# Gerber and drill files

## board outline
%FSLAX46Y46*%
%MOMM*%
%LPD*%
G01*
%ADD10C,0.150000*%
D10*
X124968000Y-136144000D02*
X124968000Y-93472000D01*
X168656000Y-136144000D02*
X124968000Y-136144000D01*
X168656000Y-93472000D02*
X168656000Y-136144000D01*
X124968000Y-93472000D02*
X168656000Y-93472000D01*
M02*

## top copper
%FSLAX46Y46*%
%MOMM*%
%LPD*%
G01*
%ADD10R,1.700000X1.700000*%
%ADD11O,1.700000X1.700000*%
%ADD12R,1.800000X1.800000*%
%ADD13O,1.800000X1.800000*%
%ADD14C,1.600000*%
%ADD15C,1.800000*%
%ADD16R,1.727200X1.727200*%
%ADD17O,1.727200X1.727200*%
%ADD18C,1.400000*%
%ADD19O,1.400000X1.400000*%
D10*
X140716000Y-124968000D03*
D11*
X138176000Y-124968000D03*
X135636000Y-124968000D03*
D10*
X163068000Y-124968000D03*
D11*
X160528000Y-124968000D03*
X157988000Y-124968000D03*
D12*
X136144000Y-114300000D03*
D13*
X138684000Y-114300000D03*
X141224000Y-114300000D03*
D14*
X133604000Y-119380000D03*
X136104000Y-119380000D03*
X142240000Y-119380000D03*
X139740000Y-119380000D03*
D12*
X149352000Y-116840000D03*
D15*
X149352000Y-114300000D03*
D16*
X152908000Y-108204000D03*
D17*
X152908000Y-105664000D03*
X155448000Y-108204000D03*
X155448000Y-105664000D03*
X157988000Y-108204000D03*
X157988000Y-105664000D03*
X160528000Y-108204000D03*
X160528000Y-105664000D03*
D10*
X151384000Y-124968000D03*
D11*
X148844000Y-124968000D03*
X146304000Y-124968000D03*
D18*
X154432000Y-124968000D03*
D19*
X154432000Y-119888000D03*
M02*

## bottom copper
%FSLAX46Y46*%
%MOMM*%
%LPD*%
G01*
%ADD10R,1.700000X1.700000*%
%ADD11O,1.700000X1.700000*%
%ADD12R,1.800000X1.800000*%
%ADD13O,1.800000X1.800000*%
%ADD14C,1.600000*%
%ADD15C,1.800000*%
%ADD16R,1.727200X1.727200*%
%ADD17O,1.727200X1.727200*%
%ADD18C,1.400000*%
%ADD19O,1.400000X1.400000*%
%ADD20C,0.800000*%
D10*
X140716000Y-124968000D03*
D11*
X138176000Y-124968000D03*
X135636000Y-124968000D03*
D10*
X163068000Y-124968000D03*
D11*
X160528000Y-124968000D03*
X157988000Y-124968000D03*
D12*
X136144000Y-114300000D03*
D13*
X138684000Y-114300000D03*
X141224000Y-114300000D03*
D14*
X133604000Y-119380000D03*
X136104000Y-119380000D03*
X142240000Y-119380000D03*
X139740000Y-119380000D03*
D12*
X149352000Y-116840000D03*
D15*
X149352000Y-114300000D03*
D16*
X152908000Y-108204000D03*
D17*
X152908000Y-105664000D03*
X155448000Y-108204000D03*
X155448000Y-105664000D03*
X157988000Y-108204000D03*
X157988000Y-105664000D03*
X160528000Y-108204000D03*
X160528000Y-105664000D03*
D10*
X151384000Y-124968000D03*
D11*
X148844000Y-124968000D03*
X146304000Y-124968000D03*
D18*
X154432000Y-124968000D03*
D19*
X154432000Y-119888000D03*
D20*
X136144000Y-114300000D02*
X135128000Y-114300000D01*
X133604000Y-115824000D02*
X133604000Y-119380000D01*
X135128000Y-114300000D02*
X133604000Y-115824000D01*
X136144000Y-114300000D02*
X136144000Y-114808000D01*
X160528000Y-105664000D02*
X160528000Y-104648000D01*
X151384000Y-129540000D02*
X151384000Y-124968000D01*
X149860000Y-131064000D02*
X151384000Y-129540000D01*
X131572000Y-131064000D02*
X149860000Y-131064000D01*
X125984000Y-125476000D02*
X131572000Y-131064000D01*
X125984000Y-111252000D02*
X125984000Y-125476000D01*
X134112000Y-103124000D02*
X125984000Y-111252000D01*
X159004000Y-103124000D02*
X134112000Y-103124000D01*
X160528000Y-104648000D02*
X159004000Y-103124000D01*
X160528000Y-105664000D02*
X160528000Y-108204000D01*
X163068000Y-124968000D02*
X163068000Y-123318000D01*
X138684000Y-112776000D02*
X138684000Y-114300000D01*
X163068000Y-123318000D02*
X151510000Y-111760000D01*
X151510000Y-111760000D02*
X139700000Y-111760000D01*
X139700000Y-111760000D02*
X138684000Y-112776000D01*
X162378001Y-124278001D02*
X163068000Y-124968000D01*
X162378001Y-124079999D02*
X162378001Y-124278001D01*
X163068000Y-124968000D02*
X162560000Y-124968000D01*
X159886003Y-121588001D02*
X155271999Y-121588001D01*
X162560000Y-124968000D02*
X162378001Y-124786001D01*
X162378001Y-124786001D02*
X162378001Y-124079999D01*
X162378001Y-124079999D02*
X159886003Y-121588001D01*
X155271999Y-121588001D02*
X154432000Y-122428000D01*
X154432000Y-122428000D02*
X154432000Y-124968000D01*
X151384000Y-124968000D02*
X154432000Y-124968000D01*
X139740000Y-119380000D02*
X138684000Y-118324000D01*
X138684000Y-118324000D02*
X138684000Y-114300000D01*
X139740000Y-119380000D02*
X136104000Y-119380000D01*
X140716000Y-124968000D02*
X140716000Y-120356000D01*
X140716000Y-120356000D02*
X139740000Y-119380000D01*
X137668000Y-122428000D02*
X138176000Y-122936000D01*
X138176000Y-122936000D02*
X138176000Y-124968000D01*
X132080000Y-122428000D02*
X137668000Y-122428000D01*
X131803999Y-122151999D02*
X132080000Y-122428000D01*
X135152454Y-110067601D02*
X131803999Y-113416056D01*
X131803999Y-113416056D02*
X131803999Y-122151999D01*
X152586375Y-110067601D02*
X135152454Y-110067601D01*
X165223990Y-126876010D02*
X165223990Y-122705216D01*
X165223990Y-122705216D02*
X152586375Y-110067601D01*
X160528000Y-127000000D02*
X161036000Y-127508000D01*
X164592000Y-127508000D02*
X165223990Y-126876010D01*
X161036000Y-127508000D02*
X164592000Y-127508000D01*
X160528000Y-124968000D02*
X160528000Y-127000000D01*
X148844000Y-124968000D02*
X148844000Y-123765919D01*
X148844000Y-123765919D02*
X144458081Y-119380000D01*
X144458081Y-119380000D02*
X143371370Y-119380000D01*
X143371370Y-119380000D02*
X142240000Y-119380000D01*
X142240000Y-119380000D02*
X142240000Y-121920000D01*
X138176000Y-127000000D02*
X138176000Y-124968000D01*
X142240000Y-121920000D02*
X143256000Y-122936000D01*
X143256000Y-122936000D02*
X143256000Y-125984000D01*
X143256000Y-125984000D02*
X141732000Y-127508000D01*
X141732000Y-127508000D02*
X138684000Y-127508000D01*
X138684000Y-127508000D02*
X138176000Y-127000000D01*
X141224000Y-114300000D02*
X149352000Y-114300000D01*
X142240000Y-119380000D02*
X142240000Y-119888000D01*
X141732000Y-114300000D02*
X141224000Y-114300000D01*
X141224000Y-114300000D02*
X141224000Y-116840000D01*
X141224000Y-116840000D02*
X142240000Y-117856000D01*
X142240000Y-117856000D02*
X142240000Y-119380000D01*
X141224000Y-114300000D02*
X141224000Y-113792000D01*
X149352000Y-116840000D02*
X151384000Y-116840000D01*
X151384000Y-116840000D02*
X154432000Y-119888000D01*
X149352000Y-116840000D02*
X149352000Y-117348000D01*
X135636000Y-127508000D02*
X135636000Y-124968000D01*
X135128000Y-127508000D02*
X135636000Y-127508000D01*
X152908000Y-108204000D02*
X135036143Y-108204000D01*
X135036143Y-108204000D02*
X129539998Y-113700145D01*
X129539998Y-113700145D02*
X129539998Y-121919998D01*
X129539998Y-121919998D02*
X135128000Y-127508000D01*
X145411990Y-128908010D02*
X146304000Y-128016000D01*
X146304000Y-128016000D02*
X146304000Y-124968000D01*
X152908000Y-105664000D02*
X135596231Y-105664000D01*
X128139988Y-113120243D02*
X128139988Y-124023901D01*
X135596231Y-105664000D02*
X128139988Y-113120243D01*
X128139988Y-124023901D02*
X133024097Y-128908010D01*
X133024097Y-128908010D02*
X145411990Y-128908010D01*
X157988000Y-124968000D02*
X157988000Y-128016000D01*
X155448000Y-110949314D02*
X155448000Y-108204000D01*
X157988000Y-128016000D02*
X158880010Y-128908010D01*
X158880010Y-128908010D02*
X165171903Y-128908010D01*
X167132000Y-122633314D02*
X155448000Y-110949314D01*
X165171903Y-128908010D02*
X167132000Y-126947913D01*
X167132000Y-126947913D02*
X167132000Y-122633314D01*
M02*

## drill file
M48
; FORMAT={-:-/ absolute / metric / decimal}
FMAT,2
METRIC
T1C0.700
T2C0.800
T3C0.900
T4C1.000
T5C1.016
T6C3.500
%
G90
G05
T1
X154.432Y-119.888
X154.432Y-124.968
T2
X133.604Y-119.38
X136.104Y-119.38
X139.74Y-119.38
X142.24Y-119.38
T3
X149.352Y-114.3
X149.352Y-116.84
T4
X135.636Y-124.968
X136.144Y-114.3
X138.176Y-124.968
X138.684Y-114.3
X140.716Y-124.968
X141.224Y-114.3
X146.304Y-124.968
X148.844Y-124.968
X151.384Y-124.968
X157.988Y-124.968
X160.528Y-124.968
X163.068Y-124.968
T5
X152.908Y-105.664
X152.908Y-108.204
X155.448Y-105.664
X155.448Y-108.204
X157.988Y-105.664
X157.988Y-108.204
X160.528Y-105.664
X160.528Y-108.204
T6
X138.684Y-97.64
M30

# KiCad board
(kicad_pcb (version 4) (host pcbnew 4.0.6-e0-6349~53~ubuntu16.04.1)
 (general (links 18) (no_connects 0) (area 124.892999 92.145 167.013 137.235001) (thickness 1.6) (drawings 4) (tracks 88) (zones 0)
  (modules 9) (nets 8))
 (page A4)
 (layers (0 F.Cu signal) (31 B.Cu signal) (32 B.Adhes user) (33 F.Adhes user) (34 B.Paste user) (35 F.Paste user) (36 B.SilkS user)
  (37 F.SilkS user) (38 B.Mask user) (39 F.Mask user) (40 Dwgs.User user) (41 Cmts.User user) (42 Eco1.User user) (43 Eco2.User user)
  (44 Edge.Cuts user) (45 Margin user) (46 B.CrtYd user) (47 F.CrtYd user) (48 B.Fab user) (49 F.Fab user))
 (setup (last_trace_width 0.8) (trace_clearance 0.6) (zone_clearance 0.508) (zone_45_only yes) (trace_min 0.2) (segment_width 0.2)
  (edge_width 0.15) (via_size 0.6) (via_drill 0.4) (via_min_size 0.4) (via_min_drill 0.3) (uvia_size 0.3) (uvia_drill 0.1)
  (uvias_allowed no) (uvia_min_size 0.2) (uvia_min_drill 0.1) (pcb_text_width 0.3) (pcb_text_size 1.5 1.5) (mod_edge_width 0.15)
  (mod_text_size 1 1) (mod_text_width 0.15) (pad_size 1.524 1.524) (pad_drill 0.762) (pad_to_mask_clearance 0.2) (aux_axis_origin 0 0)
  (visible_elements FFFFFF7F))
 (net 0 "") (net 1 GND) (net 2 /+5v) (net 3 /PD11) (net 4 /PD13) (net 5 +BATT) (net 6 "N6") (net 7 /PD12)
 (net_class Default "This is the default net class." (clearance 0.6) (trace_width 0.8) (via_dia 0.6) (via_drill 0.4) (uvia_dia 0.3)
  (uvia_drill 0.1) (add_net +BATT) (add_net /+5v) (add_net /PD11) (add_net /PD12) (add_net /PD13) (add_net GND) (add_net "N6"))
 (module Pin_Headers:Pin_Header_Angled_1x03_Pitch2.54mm (layer F.Cu) (at 140.716 124.968 270)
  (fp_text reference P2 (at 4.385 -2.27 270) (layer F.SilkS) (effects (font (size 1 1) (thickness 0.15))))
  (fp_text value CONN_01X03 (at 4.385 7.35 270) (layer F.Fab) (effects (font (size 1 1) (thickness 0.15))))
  (pad 1 thru_hole rect (at 0 0 270) (size 1.7 1.7) (drill 1) (layers *.Cu *.Mask) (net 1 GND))
  (pad 2 thru_hole oval (at 0 2.54 270) (size 1.7 1.7) (drill 1) (layers *.Cu *.Mask) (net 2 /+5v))
  (pad 3 thru_hole oval (at 0 5.08 270) (size 1.7 1.7) (drill 1) (layers *.Cu *.Mask) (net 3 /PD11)))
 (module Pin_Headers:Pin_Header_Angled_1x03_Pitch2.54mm (layer F.Cu) (at 163.068 124.968 270)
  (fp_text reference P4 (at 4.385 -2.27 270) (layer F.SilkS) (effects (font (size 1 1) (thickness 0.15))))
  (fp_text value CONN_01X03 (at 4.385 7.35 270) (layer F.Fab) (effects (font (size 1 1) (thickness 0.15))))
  (pad 1 thru_hole rect (at 0 0 270) (size 1.7 1.7) (drill 1) (layers *.Cu *.Mask) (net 1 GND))
  (pad 2 thru_hole oval (at 0 2.54 270) (size 1.7 1.7) (drill 1) (layers *.Cu *.Mask) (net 2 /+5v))
  (pad 3 thru_hole oval (at 0 5.08 270) (size 1.7 1.7) (drill 1) (layers *.Cu *.Mask) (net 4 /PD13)))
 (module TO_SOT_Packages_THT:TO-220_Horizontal (layer F.Cu) (at 136.144 114.3)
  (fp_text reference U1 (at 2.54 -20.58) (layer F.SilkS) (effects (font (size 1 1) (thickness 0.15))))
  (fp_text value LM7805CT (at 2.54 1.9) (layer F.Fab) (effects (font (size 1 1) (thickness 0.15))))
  (pad 0 np_thru_hole oval (at 2.54 -16.66) (size 3.5 3.5) (drill 3.5) (layers *.Cu *.Mask))
  (pad 1 thru_hole rect (at 0 0) (size 1.8 1.8) (drill 1) (layers *.Cu *.Mask) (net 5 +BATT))
  (pad 2 thru_hole oval (at 2.54 0) (size 1.8 1.8) (drill 1) (layers *.Cu *.Mask) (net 1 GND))
  (pad 3 thru_hole oval (at 5.08 0) (size 1.8 1.8) (drill 1) (layers *.Cu *.Mask) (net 2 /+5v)))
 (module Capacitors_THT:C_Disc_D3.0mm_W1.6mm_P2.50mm (layer F.Cu) (at 133.604 119.38)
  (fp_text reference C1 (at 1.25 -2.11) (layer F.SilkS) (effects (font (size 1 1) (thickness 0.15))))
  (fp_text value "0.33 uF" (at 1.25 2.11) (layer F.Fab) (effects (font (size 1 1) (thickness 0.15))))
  (pad 1 thru_hole circle (at 0 0) (size 1.6 1.6) (drill 0.8) (layers *.Cu *.Mask) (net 5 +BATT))
  (pad 2 thru_hole circle (at 2.5 0) (size 1.6 1.6) (drill 0.8) (layers *.Cu *.Mask) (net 1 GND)))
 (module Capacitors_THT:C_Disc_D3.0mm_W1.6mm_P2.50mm (layer F.Cu) (at 142.24 119.38 180)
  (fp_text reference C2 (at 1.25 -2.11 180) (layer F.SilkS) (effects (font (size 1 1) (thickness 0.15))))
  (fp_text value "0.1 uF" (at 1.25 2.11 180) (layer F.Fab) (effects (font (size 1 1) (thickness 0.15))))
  (pad 1 thru_hole circle (at 0 0 180) (size 1.6 1.6) (drill 0.8) (layers *.Cu *.Mask) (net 2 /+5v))
  (pad 2 thru_hole circle (at 2.5 0 180) (size 1.6 1.6) (drill 0.8) (layers *.Cu *.Mask) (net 1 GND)))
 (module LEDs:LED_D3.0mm (layer F.Cu) (at 149.352 116.84 90)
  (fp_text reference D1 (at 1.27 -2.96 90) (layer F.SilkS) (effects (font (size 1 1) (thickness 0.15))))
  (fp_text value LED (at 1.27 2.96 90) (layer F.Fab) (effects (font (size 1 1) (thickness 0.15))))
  (pad 1 thru_hole rect (at 0 0 90) (size 1.8 1.8) (drill 0.9) (layers *.Cu *.Mask) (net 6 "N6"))
  (pad 2 thru_hole circle (at 2.54 0 90) (size 1.8 1.8) (drill 0.9) (layers *.Cu *.Mask) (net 2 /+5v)))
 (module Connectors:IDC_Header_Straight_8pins (layer F.Cu) (at 152.908 108.204)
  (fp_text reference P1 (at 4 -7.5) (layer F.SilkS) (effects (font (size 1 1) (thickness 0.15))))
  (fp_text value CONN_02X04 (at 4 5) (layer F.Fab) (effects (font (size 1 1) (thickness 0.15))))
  (pad 1 thru_hole rect (at 0 0) (size 1.7272 1.7272) (drill 1.016) (layers *.Cu *.Mask) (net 3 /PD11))
  (pad 2 thru_hole oval (at 0 -2.54) (size 1.7272 1.7272) (drill 1.016) (layers *.Cu *.Mask) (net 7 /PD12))
  (pad 3 thru_hole oval (at 2.54 0) (size 1.7272 1.7272) (drill 1.016) (layers *.Cu *.Mask) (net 4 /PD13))
  (pad 4 thru_hole oval (at 2.54 -2.54) (size 1.7272 1.7272) (drill 1.016) (layers *.Cu *.Mask))
  (pad 5 thru_hole oval (at 5.08 0) (size 1.7272 1.7272) (drill 1.016) (layers *.Cu *.Mask))
  (pad 6 thru_hole oval (at 5.08 -2.54) (size 1.7272 1.7272) (drill 1.016) (layers *.Cu *.Mask))
  (pad 7 thru_hole oval (at 7.62 0) (size 1.7272 1.7272) (drill 1.016) (layers *.Cu *.Mask) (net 1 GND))
  (pad 8 thru_hole oval (at 7.62 -2.54) (size 1.7272 1.7272) (drill 1.016) (layers *.Cu *.Mask) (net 1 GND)))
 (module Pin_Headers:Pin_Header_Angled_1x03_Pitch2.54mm (layer F.Cu) (at 151.384 124.968 270)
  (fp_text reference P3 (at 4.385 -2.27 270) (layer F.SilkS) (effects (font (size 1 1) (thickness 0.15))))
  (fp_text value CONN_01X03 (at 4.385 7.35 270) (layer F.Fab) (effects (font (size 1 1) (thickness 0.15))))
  (pad 1 thru_hole rect (at 0 0 270) (size 1.7 1.7) (drill 1) (layers *.Cu *.Mask) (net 1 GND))
  (pad 2 thru_hole oval (at 0 2.54 270) (size 1.7 1.7) (drill 1) (layers *.Cu *.Mask) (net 2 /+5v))
  (pad 3 thru_hole oval (at 0 5.08 270) (size 1.7 1.7) (drill 1) (layers *.Cu *.Mask) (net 7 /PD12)))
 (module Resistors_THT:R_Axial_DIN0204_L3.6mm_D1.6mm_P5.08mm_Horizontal (layer F.Cu) (at 154.432 124.968 90)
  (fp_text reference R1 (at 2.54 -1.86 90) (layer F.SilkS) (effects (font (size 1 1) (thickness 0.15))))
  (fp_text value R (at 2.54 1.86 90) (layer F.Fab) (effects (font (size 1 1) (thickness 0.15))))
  (pad 1 thru_hole circle (at 0 0 90) (size 1.4 1.4) (drill 0.7) (layers *.Cu *.Mask) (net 1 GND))
  (pad 2 thru_hole oval (at 5.08 0 90) (size 1.4 1.4) (drill 0.7) (layers *.Cu *.Mask) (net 6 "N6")))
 (gr_line (start 124.968 136.144) (end 124.968 93.472) (angle 90) (layer Edge.Cuts) (width 0.15))
 (gr_line (start 168.656 136.144) (end 124.968 136.144) (angle 90) (layer Edge.Cuts) (width 0.15))
 (gr_line (start 168.656 93.472) (end 168.656 136.144) (angle 90) (layer Edge.Cuts) (width 0.15))
 (gr_line (start 124.968 93.472) (end 168.656 93.472) (angle 90) (layer Edge.Cuts) (width 0.15))
 (segment (start 136.144 114.3) (end 135.128 114.3) (width 0.8) (layer B.Cu) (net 5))
 (segment (start 133.604 115.824) (end 133.604 119.38) (width 0.8) (layer B.Cu) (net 5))
 (segment (start 135.128 114.3) (end 133.604 115.824) (width 0.8) (layer B.Cu) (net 5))
 (segment (start 136.144 114.3) (end 136.144 114.808) (width 0.8) (layer B.Cu) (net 5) (status 30))
 (segment (start 160.528 105.664) (end 160.528 104.648) (width 0.8) (layer B.Cu) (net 1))
 (segment (start 151.384 129.54) (end 151.384 124.968) (width 0.8) (layer B.Cu) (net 1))
 (segment (start 149.86 131.064) (end 151.384 129.54) (width 0.8) (layer B.Cu) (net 1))
 (segment (start 131.572 131.064) (end 149.86 131.064) (width 0.8) (layer B.Cu) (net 1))
 (segment (start 125.984 125.476) (end 131.572 131.064) (width 0.8) (layer B.Cu) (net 1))
 (segment (start 125.984 111.252) (end 125.984 125.476) (width 0.8) (layer B.Cu) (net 1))
 (segment (start 134.112 103.124) (end 125.984 111.252) (width 0.8) (layer B.Cu) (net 1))
 (segment (start 159.004 103.124) (end 134.112 103.124) (width 0.8) (layer B.Cu) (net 1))
 (segment (start 160.528 104.648) (end 159.004 103.124) (width 0.8) (layer B.Cu) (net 1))
 (segment (start 160.528 105.664) (end 160.528 108.204) (width 0.8) (layer B.Cu) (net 1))
 (segment (start 163.068 124.968) (end 163.068 123.318) (width 0.8) (layer B.Cu) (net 1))
 (segment (start 138.684 112.776) (end 138.684 114.3) (width 0.8) (layer B.Cu) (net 1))
 (segment (start 163.068 123.318) (end 151.51 111.76) (width 0.8) (layer B.Cu) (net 1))
 (segment (start 151.51 111.76) (end 139.7 111.76) (width 0.8) (layer B.Cu) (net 1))
 (segment (start 139.7 111.76) (end 138.684 112.776) (width 0.8) (layer B.Cu) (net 1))
 (segment (start 162.378001 124.278001) (end 163.068 124.968) (width 0.8) (layer B.Cu) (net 1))
 (segment (start 162.378001 124.079999) (end 162.378001 124.278001) (width 0.8) (layer B.Cu) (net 1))
 (segment (start 163.068 124.968) (end 162.56 124.968) (width 0.8) (layer B.Cu) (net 1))
 (segment (start 159.886003 121.588001) (end 155.271999 121.588001) (width 0.8) (layer B.Cu) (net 1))
 (segment (start 162.56 124.968) (end 162.378001 124.786001) (width 0.8) (layer B.Cu) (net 1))
 (segment (start 162.378001 124.786001) (end 162.378001 124.079999) (width 0.8) (layer B.Cu) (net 1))
 (segment (start 162.378001 124.079999) (end 159.886003 121.588001) (width 0.8) (layer B.Cu) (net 1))
 (segment (start 155.271999 121.588001) (end 154.432 122.428) (width 0.8) (layer B.Cu) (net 1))
 (segment (start 154.432 122.428) (end 154.432 124.968) (width 0.8) (layer B.Cu) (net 1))
 (segment (start 151.384 124.968) (end 154.432 124.968) (width 0.8) (layer B.Cu) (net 1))
 (segment (start 139.74 119.38) (end 138.684 118.324) (width 0.8) (layer B.Cu) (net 1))
 (segment (start 138.684 118.324) (end 138.684 114.3) (width 0.8) (layer B.Cu) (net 1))
 (segment (start 139.74 119.38) (end 136.104 119.38) (width 0.8) (layer B.Cu) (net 1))
 (segment (start 140.716 124.968) (end 140.716 120.356) (width 0.8) (layer B.Cu) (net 1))
 (segment (start 140.716 120.356) (end 139.74 119.38) (width 0.8) (layer B.Cu) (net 1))
 (segment (start 137.668 122.428) (end 138.176 122.936) (width 0.8) (layer B.Cu) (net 2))
 (segment (start 138.176 122.936) (end 138.176 124.968) (width 0.8) (layer B.Cu) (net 2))
 (segment (start 132.08 122.428) (end 137.668 122.428) (width 0.8) (layer B.Cu) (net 2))
 (segment (start 131.803999 122.151999) (end 132.08 122.428) (width 0.8) (layer B.Cu) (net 2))
 (segment (start 135.152454 110.067601) (end 131.803999 113.416056) (width 0.8) (layer B.Cu) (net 2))
 (segment (start 131.803999 113.416056) (end 131.803999 122.151999) (width 0.8) (layer B.Cu) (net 2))
 (segment (start 152.586375 110.067601) (end 135.152454 110.067601) (width 0.8) (layer B.Cu) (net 2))
 (segment (start 165.22399 126.87601) (end 165.22399 122.705216) (width 0.8) (layer B.Cu) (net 2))
 (segment (start 165.22399 122.705216) (end 152.586375 110.067601) (width 0.8) (layer B.Cu) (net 2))
 (segment (start 160.528 127) (end 161.036 127.508) (width 0.8) (layer B.Cu) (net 2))
 (segment (start 164.592 127.508) (end 165.22399 126.87601) (width 0.8) (layer B.Cu) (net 2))
 (segment (start 161.036 127.508) (end 164.592 127.508) (width 0.8) (layer B.Cu) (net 2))
 (segment (start 160.528 124.968) (end 160.528 127) (width 0.8) (layer B.Cu) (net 2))
 (segment (start 148.844 124.968) (end 148.844 123.765919) (width 0.8) (layer B.Cu) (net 2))
 (segment (start 148.844 123.765919) (end 144.458081 119.38) (width 0.8) (layer B.Cu) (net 2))
 (segment (start 144.458081 119.38) (end 143.37137 119.38) (width 0.8) (layer B.Cu) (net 2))
 (segment (start 143.37137 119.38) (end 142.24 119.38) (width 0.8) (layer B.Cu) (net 2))
 (segment (start 142.24 119.38) (end 142.24 121.92) (width 0.8) (layer B.Cu) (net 2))
 (segment (start 138.176 127) (end 138.176 124.968) (width 0.8) (layer B.Cu) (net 2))
 (segment (start 142.24 121.92) (end 143.256 122.936) (width 0.8) (layer B.Cu) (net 2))
 (segment (start 143.256 122.936) (end 143.256 125.984) (width 0.8) (layer B.Cu) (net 2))
 (segment (start 143.256 125.984) (end 141.732 127.508) (width 0.8) (layer B.Cu) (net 2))
 (segment (start 141.732 127.508) (end 138.684 127.508) (width 0.8) (layer B.Cu) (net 2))
 (segment (start 138.684 127.508) (end 138.176 127) (width 0.8) (layer B.Cu) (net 2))
 (segment (start 141.224 114.3) (end 149.352 114.3) (width 0.8) (layer B.Cu) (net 2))
 (segment (start 142.24 119.38) (end 142.24 119.888) (width 0.8) (layer B.Cu) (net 2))
 (segment (start 141.732 114.3) (end 141.224 114.3) (width 0.8) (layer B.Cu) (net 2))
 (segment (start 141.224 114.3) (end 141.224 116.84) (width 0.8) (layer B.Cu) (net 2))
 (segment (start 141.224 116.84) (end 142.24 117.856) (width 0.8) (layer B.Cu) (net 2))
 (segment (start 142.24 117.856) (end 142.24 119.38) (width 0.8) (layer B.Cu) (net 2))
 (segment (start 141.224 114.3) (end 141.224 113.792) (width 0.8) (layer B.Cu) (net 2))
 (segment (start 149.352 116.84) (end 151.384 116.84) (width 0.8) (layer B.Cu) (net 6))
 (segment (start 151.384 116.84) (end 154.432 119.888) (width 0.8) (layer B.Cu) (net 6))
 (segment (start 149.352 116.84) (end 149.352 117.348) (width 0.8) (layer B.Cu) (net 6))
 (segment (start 135.636 127.508) (end 135.636 124.968) (width 0.8) (layer B.Cu) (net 3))
 (segment (start 135.128 127.508) (end 135.636 127.508) (width 0.8) (layer B.Cu) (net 3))
 (segment (start 152.908 108.204) (end 135.036143 108.204) (width 0.8) (layer B.Cu) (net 3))
 (segment (start 135.036143 108.204) (end 129.539998 113.700145) (width 0.8) (layer B.Cu) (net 3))
 (segment (start 129.539998 113.700145) (end 129.539998 121.919998) (width 0.8) (layer B.Cu) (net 3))
 (segment (start 129.539998 121.919998) (end 135.128 127.508) (width 0.8) (layer B.Cu) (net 3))
 (segment (start 145.41199 128.90801) (end 146.304 128.016) (width 0.8) (layer B.Cu) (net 7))
 (segment (start 146.304 128.016) (end 146.304 124.968) (width 0.8) (layer B.Cu) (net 7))
 (segment (start 152.908 105.664) (end 135.596231 105.664) (width 0.8) (layer B.Cu) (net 7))
 (segment (start 128.139988 113.120243) (end 128.139988 124.023901) (width 0.8) (layer B.Cu) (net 7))
 (segment (start 135.596231 105.664) (end 128.139988 113.120243) (width 0.8) (layer B.Cu) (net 7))
 (segment (start 128.139988 124.023901) (end 133.024097 128.90801) (width 0.8) (layer B.Cu) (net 7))
 (segment (start 133.024097 128.90801) (end 145.41199 128.90801) (width 0.8) (layer B.Cu) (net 7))
 (segment (start 157.988 124.968) (end 157.988 128.016) (width 0.8) (layer B.Cu) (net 4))
 (segment (start 155.448 110.949314) (end 155.448 108.204) (width 0.8) (layer B.Cu) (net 4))
 (segment (start 157.988 128.016) (end 158.88001 128.90801) (width 0.8) (layer B.Cu) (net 4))
 (segment (start 158.88001 128.90801) (end 165.171903 128.90801) (width 0.8) (layer B.Cu) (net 4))
 (segment (start 167.132 122.633314) (end 155.448 110.949314) (width 0.8) (layer B.Cu) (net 4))
 (segment (start 165.171903 128.90801) (end 167.132 126.947913) (width 0.8) (layer B.Cu) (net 4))
 (segment (start 167.132 126.947913) (end 167.132 122.633314) (width 0.8) (layer B.Cu) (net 4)))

